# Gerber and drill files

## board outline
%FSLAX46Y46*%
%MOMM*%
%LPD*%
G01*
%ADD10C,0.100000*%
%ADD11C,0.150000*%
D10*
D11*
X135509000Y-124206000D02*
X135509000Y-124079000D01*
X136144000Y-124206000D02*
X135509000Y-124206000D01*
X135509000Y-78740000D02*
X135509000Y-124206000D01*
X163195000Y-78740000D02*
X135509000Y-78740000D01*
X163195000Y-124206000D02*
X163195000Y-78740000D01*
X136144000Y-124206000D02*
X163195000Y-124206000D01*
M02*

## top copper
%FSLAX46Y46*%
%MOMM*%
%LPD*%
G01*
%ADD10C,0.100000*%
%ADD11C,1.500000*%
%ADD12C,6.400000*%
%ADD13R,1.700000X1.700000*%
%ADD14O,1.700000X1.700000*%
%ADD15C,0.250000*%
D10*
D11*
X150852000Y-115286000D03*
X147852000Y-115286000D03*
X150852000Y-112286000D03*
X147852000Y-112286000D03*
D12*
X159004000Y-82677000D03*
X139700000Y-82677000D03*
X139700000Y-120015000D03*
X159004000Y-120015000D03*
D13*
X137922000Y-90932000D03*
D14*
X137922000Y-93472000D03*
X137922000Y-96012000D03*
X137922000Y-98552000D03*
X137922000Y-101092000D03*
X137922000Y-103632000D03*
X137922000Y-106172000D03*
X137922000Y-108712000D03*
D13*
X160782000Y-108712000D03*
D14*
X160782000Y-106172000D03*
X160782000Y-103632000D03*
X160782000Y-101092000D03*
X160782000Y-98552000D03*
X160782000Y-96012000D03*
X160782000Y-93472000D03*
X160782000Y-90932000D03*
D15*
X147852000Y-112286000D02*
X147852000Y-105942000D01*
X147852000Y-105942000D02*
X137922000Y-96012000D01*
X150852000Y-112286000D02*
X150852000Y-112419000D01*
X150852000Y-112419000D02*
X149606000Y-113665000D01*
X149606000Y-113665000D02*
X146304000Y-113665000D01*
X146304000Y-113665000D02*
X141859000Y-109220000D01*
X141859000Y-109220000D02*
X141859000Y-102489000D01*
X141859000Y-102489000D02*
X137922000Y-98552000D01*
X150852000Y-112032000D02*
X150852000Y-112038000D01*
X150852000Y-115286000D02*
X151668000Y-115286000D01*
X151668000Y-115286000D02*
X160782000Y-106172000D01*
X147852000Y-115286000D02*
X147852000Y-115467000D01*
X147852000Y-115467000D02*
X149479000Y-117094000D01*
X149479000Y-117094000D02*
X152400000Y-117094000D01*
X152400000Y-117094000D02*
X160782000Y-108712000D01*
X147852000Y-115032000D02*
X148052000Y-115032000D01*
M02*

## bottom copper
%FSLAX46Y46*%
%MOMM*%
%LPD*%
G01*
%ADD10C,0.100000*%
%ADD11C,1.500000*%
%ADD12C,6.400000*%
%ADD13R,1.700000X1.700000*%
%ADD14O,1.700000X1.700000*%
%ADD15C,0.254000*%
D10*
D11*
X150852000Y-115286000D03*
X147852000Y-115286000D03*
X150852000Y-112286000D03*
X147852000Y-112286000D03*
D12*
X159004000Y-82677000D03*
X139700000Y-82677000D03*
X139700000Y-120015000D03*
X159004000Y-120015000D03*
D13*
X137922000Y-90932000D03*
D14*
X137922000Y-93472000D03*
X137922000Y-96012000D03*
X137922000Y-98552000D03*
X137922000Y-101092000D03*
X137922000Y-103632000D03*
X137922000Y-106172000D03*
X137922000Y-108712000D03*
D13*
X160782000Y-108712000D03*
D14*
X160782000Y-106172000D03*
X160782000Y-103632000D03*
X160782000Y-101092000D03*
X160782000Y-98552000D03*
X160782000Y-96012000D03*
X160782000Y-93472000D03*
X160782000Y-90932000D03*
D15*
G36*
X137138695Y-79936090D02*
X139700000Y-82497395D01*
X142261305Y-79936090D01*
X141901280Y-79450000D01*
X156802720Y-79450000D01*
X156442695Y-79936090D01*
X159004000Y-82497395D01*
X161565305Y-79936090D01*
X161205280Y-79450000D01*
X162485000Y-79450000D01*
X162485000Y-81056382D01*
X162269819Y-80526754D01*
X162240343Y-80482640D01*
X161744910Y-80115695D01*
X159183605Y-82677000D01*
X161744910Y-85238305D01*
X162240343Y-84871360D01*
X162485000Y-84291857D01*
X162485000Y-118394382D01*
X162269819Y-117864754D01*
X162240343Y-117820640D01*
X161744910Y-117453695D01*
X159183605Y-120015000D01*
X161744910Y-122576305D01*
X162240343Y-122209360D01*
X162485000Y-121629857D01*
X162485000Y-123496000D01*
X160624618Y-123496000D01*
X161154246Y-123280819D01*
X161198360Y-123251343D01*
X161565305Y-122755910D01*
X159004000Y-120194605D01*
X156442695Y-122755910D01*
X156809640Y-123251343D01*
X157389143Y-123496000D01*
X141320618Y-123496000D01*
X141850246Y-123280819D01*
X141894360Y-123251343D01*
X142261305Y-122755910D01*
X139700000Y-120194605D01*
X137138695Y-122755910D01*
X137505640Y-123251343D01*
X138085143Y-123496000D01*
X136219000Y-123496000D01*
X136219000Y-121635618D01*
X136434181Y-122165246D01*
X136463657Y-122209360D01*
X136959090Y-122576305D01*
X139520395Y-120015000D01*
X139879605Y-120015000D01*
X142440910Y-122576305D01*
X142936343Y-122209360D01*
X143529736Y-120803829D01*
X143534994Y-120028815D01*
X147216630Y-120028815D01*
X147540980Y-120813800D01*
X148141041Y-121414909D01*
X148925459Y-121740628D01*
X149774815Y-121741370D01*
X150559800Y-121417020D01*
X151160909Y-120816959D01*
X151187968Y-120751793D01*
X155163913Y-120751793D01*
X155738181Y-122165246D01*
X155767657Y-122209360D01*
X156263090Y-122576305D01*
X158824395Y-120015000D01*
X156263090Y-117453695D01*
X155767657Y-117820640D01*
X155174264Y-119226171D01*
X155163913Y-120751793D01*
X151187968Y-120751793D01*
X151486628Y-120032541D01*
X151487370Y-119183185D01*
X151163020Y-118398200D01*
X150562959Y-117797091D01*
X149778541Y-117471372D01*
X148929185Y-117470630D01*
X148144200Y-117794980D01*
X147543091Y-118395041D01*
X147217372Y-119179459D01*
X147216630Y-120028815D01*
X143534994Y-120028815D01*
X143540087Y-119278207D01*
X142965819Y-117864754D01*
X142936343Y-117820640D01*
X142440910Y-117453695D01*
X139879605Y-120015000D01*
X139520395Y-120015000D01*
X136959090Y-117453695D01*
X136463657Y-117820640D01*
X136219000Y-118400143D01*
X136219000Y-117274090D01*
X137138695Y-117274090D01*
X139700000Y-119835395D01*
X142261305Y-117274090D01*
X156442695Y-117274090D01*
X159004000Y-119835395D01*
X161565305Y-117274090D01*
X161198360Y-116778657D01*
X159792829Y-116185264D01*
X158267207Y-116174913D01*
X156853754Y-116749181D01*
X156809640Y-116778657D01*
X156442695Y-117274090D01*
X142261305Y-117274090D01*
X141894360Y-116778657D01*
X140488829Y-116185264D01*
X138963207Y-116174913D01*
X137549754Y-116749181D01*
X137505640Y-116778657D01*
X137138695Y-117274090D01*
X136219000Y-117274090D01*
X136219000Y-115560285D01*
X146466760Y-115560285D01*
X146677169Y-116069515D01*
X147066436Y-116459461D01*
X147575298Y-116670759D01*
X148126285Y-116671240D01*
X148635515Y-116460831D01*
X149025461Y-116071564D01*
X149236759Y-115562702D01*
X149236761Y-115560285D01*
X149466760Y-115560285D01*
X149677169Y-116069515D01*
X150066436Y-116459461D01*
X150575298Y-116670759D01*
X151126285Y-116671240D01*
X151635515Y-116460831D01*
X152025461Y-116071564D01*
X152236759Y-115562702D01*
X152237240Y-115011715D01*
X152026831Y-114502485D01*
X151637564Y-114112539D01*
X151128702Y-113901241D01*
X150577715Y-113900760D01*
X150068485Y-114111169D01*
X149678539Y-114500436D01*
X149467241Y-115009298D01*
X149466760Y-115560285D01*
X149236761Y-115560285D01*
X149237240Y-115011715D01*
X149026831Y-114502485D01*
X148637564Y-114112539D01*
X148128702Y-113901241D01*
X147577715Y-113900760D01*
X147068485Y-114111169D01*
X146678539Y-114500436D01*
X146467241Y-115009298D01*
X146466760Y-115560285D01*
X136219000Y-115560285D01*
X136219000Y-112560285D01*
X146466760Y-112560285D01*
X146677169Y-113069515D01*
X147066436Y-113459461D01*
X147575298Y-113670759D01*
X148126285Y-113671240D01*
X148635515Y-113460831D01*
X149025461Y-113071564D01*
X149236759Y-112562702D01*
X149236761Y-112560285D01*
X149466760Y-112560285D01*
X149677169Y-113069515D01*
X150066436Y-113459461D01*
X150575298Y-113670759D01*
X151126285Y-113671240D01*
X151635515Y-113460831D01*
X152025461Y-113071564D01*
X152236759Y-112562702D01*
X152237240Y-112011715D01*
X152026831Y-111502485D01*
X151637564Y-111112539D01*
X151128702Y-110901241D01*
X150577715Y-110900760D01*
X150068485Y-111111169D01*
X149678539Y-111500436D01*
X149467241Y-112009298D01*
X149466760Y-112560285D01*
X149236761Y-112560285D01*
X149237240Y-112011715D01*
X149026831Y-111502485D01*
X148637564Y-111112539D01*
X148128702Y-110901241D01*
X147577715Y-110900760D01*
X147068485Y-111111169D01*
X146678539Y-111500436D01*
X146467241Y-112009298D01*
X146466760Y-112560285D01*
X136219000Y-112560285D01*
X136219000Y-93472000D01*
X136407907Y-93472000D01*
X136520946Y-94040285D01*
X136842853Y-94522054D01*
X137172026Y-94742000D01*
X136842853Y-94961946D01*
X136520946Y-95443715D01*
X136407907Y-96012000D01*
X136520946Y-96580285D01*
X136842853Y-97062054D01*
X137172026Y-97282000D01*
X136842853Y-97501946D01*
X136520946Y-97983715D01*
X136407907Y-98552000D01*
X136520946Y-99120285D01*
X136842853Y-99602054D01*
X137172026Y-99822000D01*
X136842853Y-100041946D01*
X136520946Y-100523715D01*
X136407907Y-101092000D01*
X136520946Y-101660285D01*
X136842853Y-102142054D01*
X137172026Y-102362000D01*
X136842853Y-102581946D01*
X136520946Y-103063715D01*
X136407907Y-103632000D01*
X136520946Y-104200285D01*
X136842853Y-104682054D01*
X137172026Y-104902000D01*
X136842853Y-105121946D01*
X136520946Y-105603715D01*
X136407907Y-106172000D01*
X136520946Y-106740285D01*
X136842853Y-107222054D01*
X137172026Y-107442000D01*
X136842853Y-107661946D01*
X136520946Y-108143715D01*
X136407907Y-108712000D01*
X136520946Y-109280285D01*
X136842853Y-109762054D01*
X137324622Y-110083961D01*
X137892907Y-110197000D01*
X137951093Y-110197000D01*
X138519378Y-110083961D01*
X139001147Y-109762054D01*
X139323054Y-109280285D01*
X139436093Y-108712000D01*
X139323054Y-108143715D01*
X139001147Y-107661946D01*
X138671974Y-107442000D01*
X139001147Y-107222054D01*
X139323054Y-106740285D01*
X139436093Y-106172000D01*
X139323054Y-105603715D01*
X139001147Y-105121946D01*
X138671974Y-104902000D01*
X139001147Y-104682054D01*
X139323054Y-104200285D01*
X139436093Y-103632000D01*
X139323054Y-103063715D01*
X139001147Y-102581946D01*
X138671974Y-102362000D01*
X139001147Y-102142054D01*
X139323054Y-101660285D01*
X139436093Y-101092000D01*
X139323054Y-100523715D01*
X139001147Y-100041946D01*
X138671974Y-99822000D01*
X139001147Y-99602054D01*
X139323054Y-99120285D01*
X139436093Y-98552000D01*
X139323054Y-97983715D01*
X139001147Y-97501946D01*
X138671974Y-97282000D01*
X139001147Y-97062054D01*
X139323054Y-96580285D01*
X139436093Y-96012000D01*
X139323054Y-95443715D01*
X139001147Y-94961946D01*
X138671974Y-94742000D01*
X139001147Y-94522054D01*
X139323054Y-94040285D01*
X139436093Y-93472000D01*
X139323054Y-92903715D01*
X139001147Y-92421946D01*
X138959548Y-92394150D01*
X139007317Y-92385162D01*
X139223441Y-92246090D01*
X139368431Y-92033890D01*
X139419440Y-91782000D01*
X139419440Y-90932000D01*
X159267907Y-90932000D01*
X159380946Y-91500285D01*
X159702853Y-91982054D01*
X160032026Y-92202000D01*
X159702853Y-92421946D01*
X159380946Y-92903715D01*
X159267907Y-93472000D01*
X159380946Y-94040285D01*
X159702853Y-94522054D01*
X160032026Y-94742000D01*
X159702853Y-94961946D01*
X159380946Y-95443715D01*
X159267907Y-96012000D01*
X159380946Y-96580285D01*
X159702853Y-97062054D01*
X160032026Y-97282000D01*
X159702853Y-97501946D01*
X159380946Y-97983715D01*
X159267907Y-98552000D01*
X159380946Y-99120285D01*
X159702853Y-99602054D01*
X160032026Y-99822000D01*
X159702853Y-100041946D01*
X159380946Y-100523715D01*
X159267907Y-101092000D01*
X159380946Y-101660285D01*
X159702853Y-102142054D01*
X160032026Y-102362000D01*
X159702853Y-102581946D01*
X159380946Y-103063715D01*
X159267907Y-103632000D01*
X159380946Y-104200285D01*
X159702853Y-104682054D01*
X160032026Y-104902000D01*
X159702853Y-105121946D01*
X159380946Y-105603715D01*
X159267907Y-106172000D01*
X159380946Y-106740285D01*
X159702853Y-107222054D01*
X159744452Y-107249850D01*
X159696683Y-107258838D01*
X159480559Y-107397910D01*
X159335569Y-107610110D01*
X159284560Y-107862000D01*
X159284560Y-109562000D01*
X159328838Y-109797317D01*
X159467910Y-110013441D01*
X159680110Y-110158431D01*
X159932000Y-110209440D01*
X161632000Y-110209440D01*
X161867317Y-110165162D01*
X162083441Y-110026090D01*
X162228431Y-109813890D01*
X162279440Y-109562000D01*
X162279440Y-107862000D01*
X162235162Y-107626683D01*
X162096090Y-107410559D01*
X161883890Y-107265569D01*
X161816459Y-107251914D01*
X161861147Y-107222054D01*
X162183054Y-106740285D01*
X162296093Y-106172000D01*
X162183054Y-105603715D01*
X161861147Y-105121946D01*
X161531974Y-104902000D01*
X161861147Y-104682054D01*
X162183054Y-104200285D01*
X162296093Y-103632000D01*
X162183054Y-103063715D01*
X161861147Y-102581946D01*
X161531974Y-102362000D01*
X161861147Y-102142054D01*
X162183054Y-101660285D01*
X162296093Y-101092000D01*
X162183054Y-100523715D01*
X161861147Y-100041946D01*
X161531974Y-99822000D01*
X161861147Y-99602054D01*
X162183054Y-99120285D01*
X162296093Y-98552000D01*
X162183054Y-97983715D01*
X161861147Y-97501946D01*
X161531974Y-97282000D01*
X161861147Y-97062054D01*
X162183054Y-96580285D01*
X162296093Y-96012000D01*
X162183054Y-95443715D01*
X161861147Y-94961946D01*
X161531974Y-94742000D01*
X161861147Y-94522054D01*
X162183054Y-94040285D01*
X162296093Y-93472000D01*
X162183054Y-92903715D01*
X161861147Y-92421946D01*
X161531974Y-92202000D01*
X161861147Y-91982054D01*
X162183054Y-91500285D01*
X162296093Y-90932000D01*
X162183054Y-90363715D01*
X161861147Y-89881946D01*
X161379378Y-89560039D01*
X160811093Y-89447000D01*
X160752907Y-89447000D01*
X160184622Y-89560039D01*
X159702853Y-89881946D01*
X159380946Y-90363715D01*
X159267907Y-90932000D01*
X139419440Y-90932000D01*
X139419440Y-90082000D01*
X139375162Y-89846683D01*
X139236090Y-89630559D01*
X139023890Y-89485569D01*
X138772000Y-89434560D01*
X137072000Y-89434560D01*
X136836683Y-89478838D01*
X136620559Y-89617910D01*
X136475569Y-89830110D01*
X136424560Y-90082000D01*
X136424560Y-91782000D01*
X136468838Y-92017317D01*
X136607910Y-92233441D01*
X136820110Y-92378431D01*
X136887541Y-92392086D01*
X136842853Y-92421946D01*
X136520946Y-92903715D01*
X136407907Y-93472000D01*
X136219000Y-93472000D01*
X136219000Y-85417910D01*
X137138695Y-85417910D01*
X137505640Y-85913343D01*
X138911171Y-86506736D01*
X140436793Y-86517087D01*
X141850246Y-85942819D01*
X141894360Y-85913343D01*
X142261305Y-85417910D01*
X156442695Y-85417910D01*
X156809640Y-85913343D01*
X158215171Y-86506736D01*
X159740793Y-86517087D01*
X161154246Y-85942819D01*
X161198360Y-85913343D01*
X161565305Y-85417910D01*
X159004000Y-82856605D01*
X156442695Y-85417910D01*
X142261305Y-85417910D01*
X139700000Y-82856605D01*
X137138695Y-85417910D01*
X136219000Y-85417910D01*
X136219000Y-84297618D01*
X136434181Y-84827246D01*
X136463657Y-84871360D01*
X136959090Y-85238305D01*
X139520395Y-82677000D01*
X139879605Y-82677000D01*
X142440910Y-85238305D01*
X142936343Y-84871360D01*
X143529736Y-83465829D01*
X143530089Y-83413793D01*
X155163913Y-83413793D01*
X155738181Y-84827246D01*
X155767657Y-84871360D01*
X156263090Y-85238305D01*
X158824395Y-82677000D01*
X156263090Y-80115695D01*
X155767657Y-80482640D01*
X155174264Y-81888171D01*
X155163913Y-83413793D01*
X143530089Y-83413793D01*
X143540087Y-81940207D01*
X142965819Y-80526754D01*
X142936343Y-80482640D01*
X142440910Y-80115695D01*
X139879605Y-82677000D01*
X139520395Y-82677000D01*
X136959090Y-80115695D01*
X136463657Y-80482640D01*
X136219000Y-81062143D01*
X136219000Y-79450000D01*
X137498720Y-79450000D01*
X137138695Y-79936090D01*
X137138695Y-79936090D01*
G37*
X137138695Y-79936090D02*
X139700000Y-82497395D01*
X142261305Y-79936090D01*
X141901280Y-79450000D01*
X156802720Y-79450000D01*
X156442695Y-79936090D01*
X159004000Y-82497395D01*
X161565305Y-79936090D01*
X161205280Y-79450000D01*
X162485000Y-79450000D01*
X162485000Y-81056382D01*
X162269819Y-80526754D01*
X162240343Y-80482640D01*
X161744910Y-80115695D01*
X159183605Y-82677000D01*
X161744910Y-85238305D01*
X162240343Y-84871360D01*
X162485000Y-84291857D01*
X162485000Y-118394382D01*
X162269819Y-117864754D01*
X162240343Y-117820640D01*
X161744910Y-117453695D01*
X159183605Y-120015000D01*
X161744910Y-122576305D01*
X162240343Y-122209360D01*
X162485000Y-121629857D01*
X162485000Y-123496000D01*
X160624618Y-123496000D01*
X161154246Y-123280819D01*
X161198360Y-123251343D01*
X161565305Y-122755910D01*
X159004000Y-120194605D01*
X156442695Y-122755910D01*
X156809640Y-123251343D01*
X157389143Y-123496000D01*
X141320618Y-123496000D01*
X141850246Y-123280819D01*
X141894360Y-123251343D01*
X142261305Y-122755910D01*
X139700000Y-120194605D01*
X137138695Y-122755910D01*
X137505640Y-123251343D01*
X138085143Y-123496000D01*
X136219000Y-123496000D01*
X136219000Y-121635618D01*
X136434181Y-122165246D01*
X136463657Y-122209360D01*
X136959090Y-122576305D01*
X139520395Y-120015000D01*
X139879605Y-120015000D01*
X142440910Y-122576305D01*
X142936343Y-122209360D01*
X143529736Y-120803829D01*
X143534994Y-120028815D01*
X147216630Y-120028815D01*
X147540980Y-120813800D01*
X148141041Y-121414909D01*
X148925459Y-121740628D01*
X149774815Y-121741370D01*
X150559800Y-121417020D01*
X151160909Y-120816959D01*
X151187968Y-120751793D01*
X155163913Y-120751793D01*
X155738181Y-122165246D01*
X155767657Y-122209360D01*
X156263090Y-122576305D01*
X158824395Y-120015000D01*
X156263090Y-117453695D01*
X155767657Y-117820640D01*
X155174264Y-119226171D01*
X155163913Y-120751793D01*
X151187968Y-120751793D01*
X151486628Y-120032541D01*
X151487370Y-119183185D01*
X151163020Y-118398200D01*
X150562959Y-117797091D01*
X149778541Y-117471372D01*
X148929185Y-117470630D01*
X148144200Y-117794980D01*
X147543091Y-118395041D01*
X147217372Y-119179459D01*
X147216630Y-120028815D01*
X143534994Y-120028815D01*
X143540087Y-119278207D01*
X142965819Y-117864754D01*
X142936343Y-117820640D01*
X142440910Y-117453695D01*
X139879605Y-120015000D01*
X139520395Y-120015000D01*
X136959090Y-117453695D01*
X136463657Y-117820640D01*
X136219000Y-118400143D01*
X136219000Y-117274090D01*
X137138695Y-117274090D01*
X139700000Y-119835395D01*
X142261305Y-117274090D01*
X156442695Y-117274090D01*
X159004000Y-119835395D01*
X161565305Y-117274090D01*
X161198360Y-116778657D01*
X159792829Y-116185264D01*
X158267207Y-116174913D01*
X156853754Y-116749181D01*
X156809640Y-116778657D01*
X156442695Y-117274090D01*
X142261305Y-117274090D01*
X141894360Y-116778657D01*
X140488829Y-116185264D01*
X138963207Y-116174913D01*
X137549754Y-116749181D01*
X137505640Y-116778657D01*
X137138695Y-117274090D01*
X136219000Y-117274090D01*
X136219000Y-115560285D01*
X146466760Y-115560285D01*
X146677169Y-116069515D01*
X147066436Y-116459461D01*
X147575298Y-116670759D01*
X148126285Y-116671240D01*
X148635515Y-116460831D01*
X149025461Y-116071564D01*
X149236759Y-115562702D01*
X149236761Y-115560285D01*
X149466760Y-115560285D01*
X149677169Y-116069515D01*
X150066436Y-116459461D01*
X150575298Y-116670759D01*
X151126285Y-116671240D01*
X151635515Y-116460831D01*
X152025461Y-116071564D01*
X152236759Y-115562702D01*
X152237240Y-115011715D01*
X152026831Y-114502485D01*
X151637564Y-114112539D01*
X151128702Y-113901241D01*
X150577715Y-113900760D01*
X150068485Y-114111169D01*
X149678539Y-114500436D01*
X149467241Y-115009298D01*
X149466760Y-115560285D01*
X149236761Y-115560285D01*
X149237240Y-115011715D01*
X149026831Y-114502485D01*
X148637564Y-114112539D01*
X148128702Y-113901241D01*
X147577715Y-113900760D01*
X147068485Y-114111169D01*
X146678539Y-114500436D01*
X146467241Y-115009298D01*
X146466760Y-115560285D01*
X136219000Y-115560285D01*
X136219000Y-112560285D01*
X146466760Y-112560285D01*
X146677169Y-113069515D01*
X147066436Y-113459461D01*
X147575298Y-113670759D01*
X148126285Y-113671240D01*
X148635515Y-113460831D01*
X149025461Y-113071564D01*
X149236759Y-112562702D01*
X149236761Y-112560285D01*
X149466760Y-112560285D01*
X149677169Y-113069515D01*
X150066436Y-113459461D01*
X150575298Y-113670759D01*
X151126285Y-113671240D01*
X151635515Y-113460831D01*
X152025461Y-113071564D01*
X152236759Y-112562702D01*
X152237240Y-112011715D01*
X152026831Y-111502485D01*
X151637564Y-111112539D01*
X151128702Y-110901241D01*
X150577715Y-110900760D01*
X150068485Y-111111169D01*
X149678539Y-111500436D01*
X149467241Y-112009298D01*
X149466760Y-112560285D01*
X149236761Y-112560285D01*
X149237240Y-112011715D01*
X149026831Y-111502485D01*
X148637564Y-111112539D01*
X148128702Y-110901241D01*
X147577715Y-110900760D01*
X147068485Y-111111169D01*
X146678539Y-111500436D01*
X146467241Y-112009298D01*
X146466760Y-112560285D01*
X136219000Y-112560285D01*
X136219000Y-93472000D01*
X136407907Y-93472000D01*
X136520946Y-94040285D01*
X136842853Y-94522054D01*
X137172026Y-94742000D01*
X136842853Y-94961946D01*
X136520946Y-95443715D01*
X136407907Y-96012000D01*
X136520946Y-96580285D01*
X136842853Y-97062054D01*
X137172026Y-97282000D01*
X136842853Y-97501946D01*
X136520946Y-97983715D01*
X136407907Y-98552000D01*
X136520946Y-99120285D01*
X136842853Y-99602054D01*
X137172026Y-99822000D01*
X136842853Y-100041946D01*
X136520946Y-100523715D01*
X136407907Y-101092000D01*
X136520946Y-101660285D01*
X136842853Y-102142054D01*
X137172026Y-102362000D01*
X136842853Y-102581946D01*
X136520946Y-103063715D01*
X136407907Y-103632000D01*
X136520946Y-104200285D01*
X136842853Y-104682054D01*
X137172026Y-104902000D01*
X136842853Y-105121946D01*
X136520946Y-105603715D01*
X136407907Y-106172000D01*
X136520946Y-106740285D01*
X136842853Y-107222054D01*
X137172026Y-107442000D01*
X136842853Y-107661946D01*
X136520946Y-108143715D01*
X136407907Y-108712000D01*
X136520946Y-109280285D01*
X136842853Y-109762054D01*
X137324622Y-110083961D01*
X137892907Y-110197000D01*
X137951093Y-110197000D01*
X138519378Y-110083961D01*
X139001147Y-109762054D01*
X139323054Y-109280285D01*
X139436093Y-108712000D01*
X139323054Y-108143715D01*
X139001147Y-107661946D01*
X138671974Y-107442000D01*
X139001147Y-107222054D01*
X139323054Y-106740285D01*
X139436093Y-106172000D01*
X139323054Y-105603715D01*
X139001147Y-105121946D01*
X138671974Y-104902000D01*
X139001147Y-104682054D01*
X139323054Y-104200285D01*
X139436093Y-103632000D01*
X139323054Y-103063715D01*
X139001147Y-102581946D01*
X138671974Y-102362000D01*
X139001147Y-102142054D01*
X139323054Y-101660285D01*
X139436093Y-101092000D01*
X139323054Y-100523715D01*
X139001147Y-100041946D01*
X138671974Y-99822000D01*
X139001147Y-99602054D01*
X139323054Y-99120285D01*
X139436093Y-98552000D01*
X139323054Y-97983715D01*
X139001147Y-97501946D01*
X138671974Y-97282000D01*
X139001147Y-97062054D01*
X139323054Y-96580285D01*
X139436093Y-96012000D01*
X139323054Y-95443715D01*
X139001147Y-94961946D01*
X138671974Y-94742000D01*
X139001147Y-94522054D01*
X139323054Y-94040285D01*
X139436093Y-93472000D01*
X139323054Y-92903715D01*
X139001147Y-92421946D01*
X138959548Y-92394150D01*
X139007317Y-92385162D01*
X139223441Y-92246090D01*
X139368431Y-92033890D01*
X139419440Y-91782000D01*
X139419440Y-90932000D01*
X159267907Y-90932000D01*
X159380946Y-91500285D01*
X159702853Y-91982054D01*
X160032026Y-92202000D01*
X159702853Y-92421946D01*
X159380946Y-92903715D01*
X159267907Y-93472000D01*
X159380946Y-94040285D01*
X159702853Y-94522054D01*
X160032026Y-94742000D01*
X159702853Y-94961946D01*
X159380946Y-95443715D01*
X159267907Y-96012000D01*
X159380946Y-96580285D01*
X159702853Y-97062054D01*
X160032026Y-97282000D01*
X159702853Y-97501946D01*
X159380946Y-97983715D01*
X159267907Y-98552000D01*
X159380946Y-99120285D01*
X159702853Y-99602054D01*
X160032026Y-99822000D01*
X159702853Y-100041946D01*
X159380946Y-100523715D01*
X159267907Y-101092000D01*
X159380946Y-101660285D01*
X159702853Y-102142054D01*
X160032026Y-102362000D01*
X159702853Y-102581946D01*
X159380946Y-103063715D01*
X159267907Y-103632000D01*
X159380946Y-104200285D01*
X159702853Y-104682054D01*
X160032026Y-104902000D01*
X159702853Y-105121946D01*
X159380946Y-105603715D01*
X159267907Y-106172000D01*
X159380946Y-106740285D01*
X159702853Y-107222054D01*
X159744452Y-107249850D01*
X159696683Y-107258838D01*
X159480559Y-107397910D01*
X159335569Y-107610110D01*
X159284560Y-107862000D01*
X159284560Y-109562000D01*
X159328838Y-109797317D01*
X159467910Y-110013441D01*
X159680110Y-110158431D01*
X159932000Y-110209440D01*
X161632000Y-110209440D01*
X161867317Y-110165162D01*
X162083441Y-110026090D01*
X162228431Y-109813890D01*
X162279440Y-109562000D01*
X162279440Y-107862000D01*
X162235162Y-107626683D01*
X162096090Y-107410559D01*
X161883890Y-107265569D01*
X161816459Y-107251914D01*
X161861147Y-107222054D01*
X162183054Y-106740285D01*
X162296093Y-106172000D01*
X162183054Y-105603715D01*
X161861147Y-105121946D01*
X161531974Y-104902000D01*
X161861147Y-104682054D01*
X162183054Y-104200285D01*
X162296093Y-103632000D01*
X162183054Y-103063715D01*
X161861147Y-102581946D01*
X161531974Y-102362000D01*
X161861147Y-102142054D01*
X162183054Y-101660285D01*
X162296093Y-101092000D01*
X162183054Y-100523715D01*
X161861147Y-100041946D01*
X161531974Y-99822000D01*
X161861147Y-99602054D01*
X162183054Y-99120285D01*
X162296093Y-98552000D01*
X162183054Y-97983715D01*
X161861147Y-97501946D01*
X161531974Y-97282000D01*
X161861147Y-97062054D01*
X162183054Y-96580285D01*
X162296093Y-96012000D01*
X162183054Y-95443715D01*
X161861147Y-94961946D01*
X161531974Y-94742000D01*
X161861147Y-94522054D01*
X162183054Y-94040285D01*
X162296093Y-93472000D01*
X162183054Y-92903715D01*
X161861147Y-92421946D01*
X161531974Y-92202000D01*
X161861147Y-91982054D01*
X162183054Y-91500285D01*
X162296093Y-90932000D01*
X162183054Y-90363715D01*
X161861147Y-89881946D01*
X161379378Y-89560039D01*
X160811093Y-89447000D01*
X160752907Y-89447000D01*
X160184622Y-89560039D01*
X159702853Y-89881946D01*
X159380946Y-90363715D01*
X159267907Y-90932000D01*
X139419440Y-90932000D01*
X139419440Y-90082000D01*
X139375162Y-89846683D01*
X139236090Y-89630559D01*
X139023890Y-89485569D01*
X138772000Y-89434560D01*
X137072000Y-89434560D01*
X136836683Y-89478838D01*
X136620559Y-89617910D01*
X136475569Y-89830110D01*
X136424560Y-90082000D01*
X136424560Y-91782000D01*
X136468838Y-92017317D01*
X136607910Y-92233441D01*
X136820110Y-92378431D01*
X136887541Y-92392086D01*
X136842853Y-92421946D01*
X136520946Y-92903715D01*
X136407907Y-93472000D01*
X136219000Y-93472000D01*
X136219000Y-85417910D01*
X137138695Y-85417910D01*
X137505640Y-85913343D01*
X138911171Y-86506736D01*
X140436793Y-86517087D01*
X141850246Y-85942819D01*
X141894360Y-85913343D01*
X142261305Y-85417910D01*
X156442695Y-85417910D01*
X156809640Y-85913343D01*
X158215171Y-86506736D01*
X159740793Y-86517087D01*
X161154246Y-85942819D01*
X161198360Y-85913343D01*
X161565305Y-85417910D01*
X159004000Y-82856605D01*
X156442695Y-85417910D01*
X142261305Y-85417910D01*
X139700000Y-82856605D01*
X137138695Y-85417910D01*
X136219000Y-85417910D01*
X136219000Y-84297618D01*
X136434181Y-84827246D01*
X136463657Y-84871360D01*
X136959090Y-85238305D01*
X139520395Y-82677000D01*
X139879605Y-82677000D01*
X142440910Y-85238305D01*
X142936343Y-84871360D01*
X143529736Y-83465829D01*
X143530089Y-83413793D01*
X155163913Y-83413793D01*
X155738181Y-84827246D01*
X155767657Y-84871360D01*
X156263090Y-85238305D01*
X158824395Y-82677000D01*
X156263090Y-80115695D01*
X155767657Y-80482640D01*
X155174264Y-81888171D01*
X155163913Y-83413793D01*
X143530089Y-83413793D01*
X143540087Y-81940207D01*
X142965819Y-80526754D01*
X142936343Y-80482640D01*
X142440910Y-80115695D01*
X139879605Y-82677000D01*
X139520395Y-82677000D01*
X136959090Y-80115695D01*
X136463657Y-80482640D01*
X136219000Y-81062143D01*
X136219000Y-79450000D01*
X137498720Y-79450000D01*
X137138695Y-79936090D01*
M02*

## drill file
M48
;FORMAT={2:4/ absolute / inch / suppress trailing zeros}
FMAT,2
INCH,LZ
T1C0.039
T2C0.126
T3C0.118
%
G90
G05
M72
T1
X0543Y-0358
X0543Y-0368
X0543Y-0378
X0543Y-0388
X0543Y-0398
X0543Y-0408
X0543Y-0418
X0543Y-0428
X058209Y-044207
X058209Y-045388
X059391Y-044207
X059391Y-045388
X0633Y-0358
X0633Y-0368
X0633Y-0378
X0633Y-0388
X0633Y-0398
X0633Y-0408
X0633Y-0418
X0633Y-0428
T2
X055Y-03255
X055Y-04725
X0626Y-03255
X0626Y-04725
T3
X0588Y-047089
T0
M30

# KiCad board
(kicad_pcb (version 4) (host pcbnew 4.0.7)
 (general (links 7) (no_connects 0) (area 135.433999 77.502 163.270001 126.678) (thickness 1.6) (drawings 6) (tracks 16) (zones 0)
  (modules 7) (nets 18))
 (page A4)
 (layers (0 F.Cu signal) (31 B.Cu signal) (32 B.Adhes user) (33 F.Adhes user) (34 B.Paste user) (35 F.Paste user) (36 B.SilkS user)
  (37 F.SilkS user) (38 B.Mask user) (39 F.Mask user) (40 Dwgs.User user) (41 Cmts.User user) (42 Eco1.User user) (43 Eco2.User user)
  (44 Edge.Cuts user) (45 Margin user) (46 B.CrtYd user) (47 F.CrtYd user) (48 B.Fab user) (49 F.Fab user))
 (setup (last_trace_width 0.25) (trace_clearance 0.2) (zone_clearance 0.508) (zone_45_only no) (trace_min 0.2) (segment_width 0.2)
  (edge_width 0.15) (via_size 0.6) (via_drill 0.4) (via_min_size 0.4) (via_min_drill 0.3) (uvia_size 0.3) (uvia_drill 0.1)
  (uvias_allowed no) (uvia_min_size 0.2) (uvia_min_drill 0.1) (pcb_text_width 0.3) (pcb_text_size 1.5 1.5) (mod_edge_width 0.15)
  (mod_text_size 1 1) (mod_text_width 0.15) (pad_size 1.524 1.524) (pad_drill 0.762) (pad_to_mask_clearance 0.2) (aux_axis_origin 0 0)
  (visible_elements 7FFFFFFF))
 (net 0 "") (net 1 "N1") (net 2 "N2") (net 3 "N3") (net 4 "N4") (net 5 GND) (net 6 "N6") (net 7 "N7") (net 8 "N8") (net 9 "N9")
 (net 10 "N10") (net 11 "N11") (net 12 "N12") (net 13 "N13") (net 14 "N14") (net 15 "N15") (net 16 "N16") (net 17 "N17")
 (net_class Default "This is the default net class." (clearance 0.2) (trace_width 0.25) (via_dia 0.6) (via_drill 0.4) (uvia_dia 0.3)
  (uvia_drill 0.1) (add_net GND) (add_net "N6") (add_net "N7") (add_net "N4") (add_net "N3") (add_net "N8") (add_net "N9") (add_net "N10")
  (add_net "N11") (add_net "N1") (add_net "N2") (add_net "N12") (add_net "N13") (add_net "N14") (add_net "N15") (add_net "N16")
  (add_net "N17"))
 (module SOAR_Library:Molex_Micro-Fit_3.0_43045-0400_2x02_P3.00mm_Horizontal (layer F.Cu) (at 149.352 124.206)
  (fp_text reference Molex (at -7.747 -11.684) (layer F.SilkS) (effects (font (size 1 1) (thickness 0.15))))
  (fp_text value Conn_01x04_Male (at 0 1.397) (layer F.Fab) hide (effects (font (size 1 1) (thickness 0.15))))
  (pad "" np_thru_hole circle (at 0 -4.6 180) (size 3 3) (drill 3) (layers *.Cu *.Mask))
  (pad 1 thru_hole circle (at 1.5 -8.92 180) (size 1.5 1.5) (drill 1) (layers *.Cu *.Mask) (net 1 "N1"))
  (pad 2 thru_hole circle (at -1.5 -8.92 180) (size 1.5 1.5) (drill 1) (layers *.Cu *.Mask) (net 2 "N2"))
  (pad 3 thru_hole circle (at 1.5 -11.92 180) (size 1.5 1.5) (drill 1) (layers *.Cu *.Mask) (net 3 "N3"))
  (pad 4 thru_hole circle (at -1.5 -11.92 180) (size 1.5 1.5) (drill 1) (layers *.Cu *.Mask) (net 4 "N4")))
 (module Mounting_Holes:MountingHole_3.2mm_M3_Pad (layer F.Cu) (at 159.004 82.677)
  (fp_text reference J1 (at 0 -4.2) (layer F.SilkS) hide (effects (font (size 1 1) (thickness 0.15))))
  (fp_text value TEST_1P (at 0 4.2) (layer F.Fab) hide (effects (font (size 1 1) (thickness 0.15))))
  (pad 1 thru_hole circle (at 0 0) (size 6.4 6.4) (drill 3.2) (layers *.Cu *.Mask) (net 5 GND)))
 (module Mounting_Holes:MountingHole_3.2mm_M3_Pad (layer F.Cu) (at 139.7 82.677)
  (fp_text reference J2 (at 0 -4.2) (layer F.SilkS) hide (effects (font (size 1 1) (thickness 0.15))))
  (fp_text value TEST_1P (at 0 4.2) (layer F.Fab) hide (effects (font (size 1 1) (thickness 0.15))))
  (pad 1 thru_hole circle (at 0 0) (size 6.4 6.4) (drill 3.2) (layers *.Cu *.Mask) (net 5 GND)))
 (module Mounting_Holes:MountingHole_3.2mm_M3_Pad (layer F.Cu) (at 139.7 120.015)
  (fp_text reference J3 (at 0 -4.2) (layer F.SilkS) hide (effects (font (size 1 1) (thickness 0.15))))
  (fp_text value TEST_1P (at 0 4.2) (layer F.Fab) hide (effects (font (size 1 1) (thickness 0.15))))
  (pad 1 thru_hole circle (at 0 0) (size 6.4 6.4) (drill 3.2) (layers *.Cu *.Mask) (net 5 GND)))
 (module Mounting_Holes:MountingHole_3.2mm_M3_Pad (layer F.Cu) (at 159.004 120.015)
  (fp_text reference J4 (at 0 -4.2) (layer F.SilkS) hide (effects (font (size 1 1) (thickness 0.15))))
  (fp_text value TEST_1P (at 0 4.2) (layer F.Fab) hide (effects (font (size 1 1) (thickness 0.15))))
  (pad 1 thru_hole circle (at 0 0) (size 6.4 6.4) (drill 3.2) (layers *.Cu *.Mask) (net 5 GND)))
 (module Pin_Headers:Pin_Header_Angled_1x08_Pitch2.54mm (layer F.Cu) (at 137.922 90.932)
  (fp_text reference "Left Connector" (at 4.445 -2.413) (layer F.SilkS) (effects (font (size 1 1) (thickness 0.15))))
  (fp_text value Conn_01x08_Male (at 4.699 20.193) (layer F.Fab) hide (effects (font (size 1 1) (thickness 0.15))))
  (pad 1 thru_hole rect (at 0 0) (size 1.7 1.7) (drill 1) (layers *.Cu *.Mask) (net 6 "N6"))
  (pad 2 thru_hole oval (at 0 2.54) (size 1.7 1.7) (drill 1) (layers *.Cu *.Mask) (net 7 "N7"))
  (pad 3 thru_hole oval (at 0 5.08) (size 1.7 1.7) (drill 1) (layers *.Cu *.Mask) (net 4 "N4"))
  (pad 4 thru_hole oval (at 0 7.62) (size 1.7 1.7) (drill 1) (layers *.Cu *.Mask) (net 3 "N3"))
  (pad 5 thru_hole oval (at 0 10.16) (size 1.7 1.7) (drill 1) (layers *.Cu *.Mask) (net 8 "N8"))
  (pad 6 thru_hole oval (at 0 12.7) (size 1.7 1.7) (drill 1) (layers *.Cu *.Mask) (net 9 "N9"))
  (pad 7 thru_hole oval (at 0 15.24) (size 1.7 1.7) (drill 1) (layers *.Cu *.Mask) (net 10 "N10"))
  (pad 8 thru_hole oval (at 0 17.78) (size 1.7 1.7) (drill 1) (layers *.Cu *.Mask) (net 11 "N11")))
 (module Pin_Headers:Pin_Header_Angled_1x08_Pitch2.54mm (layer F.Cu) (at 160.782 108.712 180)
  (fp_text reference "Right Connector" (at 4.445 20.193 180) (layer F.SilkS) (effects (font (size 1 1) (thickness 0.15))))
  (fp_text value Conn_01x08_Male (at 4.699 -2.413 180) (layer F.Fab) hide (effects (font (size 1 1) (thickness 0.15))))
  (pad 1 thru_hole rect (at 0 0 180) (size 1.7 1.7) (drill 1) (layers *.Cu *.Mask) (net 2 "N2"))
  (pad 2 thru_hole oval (at 0 2.54 180) (size 1.7 1.7) (drill 1) (layers *.Cu *.Mask) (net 1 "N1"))
  (pad 3 thru_hole oval (at 0 5.08 180) (size 1.7 1.7) (drill 1) (layers *.Cu *.Mask) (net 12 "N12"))
  (pad 4 thru_hole oval (at 0 7.62 180) (size 1.7 1.7) (drill 1) (layers *.Cu *.Mask) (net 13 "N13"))
  (pad 5 thru_hole oval (at 0 10.16 180) (size 1.7 1.7) (drill 1) (layers *.Cu *.Mask) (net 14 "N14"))
  (pad 6 thru_hole oval (at 0 12.7 180) (size 1.7 1.7) (drill 1) (layers *.Cu *.Mask) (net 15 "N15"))
  (pad 7 thru_hole oval (at 0 15.24 180) (size 1.7 1.7) (drill 1) (layers *.Cu *.Mask) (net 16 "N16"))
  (pad 8 thru_hole oval (at 0 17.78 180) (size 1.7 1.7) (drill 1) (layers *.Cu *.Mask) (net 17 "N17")))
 (gr_line (start 135.509 124.206) (end 135.509 124.079) (angle 90) (layer Edge.Cuts) (width 0.15))
 (gr_line (start 136.144 124.206) (end 135.509 124.206) (angle 90) (layer Edge.Cuts) (width 0.15))
 (gr_line (start 135.509 78.74) (end 135.509 124.206) (angle 90) (layer Edge.Cuts) (width 0.15))
 (gr_line (start 163.195 78.74) (end 135.509 78.74) (angle 90) (layer Edge.Cuts) (width 0.15))
 (gr_line (start 163.195 124.206) (end 163.195 78.74) (angle 90) (layer Edge.Cuts) (width 0.15))
 (gr_line (start 136.144 124.206) (end 163.195 124.206) (angle 90) (layer Edge.Cuts) (width 0.15))
 (segment (start 147.852 112.286) (end 147.852 105.942) (width 0.25) (layer F.Cu) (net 4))
 (segment (start 147.852 105.942) (end 137.922 96.012) (width 0.25) (layer F.Cu) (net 4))
 (segment (start 150.852 112.286) (end 150.852 112.419) (width 0.25) (layer F.Cu) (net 3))
 (segment (start 150.852 112.419) (end 149.606 113.665) (width 0.25) (layer F.Cu) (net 3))
 (segment (start 149.606 113.665) (end 146.304 113.665) (width 0.25) (layer F.Cu) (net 3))
 (segment (start 146.304 113.665) (end 141.859 109.22) (width 0.25) (layer F.Cu) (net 3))
 (segment (start 141.859 109.22) (end 141.859 102.489) (width 0.25) (layer F.Cu) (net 3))
 (segment (start 141.859 102.489) (end 137.922 98.552) (width 0.25) (layer F.Cu) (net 3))
 (segment (start 150.852 112.032) (end 150.852 112.038) (width 0.25) (layer F.Cu) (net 3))
 (segment (start 150.852 115.286) (end 151.668 115.286) (width 0.25) (layer F.Cu) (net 1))
 (segment (start 151.668 115.286) (end 160.782 106.172) (width 0.25) (layer F.Cu) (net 1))
 (segment (start 147.852 115.286) (end 147.852 115.467) (width 0.25) (layer F.Cu) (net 2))
 (segment (start 147.852 115.467) (end 149.479 117.094) (width 0.25) (layer F.Cu) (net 2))
 (segment (start 149.479 117.094) (end 152.4 117.094) (width 0.25) (layer F.Cu) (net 2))
 (segment (start 152.4 117.094) (end 160.782 108.712) (width 0.25) (layer F.Cu) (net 2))
 (segment (start 147.852 115.032) (end 148.052 115.032) (width 0.25) (layer F.Cu) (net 2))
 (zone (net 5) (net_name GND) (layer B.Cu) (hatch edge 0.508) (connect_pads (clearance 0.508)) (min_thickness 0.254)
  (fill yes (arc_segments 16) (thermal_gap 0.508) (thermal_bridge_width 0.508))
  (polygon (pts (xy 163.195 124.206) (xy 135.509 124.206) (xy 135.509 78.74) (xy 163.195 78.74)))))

